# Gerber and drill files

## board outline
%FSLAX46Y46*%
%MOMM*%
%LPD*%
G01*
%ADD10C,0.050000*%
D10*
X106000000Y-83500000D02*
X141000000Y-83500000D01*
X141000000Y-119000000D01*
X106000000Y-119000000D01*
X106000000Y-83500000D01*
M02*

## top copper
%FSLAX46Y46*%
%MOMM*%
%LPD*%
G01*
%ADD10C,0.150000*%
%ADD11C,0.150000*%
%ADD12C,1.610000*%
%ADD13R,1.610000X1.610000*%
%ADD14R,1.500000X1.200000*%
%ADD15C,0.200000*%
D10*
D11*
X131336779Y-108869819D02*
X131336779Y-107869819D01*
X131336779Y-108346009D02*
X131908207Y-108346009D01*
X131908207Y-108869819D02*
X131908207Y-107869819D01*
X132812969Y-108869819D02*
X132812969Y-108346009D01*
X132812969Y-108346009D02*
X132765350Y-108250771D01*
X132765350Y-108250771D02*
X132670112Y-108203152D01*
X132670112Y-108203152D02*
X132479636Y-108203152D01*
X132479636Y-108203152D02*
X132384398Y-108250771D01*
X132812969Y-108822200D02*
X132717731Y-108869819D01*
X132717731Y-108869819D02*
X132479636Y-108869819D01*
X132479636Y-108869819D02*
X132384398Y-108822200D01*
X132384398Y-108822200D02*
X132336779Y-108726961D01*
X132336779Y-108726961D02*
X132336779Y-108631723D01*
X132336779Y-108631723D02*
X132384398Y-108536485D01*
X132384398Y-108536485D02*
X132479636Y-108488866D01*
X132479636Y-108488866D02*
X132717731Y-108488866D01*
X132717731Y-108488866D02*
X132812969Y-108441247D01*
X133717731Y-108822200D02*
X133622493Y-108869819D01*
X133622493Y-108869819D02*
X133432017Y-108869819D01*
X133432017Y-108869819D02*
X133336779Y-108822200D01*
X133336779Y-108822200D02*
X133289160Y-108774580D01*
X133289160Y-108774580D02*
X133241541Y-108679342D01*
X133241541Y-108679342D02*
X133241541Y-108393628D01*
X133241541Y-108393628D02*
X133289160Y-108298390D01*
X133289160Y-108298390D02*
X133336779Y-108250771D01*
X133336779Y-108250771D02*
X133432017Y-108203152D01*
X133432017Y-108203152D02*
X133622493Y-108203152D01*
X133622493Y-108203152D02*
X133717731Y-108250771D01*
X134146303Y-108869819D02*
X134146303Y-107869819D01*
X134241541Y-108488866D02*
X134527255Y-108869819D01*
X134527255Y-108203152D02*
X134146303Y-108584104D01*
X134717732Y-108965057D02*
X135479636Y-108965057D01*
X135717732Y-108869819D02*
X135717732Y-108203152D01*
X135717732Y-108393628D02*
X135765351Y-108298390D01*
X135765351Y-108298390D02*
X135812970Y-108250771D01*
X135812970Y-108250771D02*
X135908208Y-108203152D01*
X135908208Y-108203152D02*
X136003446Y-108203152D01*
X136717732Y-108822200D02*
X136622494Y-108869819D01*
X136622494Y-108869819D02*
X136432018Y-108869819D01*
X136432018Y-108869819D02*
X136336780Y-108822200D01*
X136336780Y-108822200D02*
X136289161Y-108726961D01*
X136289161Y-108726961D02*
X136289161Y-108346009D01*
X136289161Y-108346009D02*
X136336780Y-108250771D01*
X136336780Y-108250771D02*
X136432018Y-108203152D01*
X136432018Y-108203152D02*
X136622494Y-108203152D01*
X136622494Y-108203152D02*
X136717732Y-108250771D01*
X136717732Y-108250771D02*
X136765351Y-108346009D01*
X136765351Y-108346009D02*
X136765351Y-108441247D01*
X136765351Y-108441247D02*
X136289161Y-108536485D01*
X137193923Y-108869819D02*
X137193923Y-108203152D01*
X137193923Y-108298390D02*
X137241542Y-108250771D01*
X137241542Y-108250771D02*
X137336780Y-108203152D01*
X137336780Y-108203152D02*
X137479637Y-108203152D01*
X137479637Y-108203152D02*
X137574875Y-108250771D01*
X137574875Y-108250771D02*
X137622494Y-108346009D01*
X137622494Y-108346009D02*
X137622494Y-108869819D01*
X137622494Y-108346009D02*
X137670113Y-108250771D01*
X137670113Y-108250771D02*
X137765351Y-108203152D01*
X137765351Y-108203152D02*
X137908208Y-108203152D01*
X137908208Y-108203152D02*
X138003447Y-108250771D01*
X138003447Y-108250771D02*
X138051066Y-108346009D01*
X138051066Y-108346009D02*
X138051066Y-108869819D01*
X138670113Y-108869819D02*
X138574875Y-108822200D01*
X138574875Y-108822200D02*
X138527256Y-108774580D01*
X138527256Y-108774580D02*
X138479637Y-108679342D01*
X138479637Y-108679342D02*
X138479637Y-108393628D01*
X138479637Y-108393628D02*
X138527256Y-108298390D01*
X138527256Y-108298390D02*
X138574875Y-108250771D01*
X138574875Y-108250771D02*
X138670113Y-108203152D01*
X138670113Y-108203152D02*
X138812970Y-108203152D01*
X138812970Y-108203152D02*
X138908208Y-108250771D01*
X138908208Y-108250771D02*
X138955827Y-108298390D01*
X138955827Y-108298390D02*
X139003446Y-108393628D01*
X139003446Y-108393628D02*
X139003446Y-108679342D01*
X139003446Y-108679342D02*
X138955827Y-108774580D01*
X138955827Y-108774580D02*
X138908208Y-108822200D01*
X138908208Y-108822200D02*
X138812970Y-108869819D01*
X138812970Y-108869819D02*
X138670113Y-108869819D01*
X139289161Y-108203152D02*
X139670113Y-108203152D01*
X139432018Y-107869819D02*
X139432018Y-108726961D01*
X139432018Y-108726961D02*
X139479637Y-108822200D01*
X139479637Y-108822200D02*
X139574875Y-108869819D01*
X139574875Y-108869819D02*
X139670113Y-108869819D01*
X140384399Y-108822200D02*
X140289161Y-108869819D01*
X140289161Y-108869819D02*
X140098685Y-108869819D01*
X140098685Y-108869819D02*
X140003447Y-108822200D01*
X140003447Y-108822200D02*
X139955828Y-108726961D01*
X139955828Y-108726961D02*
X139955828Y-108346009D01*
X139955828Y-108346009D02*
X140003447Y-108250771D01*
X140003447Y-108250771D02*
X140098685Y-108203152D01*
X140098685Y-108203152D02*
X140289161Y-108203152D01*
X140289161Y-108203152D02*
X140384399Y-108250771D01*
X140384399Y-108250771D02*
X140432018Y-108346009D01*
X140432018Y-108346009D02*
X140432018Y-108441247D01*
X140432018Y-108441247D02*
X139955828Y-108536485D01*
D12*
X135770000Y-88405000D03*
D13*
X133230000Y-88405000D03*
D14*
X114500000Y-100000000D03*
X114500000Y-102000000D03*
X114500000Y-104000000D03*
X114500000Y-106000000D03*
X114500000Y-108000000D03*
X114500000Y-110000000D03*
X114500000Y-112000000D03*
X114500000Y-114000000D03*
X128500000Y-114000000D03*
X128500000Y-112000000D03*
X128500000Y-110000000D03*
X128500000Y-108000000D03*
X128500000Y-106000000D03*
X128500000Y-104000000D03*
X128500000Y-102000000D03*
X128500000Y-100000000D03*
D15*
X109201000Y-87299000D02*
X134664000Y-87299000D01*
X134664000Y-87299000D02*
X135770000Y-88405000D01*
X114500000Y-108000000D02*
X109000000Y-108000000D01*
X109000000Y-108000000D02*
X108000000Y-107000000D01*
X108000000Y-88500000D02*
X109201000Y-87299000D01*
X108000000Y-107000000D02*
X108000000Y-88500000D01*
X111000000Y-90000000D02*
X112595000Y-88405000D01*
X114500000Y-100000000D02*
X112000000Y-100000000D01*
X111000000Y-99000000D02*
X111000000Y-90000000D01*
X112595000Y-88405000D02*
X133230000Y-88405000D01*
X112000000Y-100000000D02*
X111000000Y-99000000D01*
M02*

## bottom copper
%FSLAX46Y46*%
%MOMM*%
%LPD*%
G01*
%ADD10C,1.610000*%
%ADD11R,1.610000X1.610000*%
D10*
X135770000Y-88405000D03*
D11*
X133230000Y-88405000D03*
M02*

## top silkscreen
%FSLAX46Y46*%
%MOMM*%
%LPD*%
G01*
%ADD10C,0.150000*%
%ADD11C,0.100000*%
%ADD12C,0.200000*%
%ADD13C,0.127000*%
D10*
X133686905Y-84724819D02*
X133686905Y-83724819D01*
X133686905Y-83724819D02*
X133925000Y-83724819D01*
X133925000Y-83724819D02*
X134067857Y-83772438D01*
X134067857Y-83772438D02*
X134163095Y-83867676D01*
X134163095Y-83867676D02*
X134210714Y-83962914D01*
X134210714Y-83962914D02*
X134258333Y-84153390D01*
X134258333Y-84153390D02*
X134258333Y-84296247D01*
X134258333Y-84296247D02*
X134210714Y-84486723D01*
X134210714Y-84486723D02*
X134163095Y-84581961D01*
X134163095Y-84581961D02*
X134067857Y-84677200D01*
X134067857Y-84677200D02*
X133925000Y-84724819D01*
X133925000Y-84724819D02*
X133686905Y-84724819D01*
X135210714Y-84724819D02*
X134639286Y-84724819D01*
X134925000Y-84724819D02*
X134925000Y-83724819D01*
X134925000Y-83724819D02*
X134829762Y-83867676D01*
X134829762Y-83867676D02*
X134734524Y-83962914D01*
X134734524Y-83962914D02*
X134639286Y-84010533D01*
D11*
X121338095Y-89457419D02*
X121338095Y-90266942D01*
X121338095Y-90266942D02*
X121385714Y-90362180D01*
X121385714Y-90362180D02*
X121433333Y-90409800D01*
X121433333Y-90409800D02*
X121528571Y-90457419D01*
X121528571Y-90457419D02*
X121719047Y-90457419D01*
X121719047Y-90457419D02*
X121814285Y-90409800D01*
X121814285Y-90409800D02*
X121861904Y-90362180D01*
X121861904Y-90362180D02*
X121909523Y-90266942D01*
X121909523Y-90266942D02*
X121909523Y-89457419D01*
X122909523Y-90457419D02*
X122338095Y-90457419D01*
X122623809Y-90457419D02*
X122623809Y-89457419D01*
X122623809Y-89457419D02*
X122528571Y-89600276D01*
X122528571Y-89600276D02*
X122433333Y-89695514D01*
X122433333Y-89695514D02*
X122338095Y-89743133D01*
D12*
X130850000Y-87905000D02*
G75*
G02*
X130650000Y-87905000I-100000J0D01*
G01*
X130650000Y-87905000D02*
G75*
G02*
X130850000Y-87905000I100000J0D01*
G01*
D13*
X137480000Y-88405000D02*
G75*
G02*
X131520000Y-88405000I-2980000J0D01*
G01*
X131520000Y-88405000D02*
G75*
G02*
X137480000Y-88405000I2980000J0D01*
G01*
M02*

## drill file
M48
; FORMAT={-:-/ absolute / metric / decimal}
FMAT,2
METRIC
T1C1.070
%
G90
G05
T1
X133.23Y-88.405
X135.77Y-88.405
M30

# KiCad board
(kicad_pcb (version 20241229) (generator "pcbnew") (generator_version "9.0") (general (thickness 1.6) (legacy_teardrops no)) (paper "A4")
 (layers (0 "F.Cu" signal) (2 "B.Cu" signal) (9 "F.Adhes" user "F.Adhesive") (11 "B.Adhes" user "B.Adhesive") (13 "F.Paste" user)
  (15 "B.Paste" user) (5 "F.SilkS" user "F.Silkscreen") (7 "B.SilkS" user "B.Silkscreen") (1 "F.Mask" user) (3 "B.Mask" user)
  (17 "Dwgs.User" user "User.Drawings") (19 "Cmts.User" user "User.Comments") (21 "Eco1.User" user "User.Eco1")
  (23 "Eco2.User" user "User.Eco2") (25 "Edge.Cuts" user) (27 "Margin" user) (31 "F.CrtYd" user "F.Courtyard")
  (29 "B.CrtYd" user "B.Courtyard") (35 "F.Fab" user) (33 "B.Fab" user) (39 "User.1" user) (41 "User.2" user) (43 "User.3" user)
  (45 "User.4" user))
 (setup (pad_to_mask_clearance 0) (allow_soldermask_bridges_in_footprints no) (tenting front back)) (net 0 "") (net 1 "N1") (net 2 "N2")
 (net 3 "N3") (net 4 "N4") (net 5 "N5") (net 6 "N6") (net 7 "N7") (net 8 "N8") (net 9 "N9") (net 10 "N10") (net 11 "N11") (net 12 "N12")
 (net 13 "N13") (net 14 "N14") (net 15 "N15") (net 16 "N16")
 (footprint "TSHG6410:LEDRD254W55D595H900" (layer "F.Cu") (at 134.5 88.405)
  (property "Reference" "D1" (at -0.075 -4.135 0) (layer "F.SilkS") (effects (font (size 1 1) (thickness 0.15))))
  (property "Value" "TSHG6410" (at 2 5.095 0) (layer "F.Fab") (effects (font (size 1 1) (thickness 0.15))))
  (fp_circle (center -3.75 -0.5) (end -3.65 -0.5) (stroke (width 0.2) (type solid)) (fill no) (layer "F.SilkS"))
  (fp_circle (center 0 0) (end 2.98 0) (stroke (width 0.127) (type solid)) (fill no) (layer "F.SilkS"))
  (pad "A" thru_hole circle (at 1.27 0) (size 1.61 1.61) (drill 1.07) (layers "*.Cu" "*.Mask") (remove_unused_layers no) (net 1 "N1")
   (solder_mask_margin 0.102))
  (pad "C" thru_hole rect (at -1.27 0) (size 1.61 1.61) (drill 1.07) (layers "*.Cu" "*.Mask") (remove_unused_layers no) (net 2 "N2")
   (solder_mask_margin 0.102)))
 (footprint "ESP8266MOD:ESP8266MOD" (layer "F.Cu") (at 108.3 85.4)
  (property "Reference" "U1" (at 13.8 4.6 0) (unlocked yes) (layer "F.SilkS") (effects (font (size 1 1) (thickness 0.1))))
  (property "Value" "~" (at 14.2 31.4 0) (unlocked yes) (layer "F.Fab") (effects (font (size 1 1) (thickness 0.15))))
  (pad "1" smd rect (at 6.2 14.6) (size 1.5 1.2) (layers "F.Cu" "F.Mask" "F.Paste") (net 2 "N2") (thermal_bridge_angle 45))
  (pad "2" smd rect (at 6.2 16.6) (size 1.5 1.2) (layers "F.Cu" "F.Mask" "F.Paste") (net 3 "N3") (thermal_bridge_angle 45))
  (pad "3" smd rect (at 6.2 18.6) (size 1.5 1.2) (layers "F.Cu" "F.Mask" "F.Paste") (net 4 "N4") (thermal_bridge_angle 45))
  (pad "4" smd rect (at 6.2 20.6) (size 1.5 1.2) (layers "F.Cu" "F.Mask" "F.Paste") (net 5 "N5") (thermal_bridge_angle 45))
  (pad "5" smd rect (at 6.2 22.6) (size 1.5 1.2) (layers "F.Cu" "F.Mask" "F.Paste") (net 1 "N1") (thermal_bridge_angle 45))
  (pad "6" smd rect (at 6.2 24.6) (size 1.5 1.2) (layers "F.Cu" "F.Mask" "F.Paste") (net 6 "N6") (thermal_bridge_angle 45))
  (pad "7" smd rect (at 6.2 26.6) (size 1.5 1.2) (layers "F.Cu" "F.Mask" "F.Paste") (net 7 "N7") (thermal_bridge_angle 45))
  (pad "8" smd rect (at 6.2 28.6) (size 1.5 1.2) (layers "F.Cu" "F.Mask" "F.Paste") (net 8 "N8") (thermal_bridge_angle 45))
  (pad "9" smd rect (at 20.2 28.6) (size 1.5 1.2) (layers "F.Cu" "F.Mask" "F.Paste") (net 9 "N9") (thermal_bridge_angle 45))
  (pad "10" smd rect (at 20.2 26.6) (size 1.5 1.2) (layers "F.Cu" "F.Mask" "F.Paste") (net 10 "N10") (thermal_bridge_angle 45))
  (pad "11" smd rect (at 20.2 24.6) (size 1.5 1.2) (layers "F.Cu" "F.Mask" "F.Paste") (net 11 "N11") (thermal_bridge_angle 45))
  (pad "12" smd rect (at 20.2 22.6) (size 1.5 1.2) (layers "F.Cu" "F.Mask" "F.Paste") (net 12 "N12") (thermal_bridge_angle 45))
  (pad "13" smd rect (at 20.2 20.6) (size 1.5 1.2) (layers "F.Cu" "F.Mask" "F.Paste") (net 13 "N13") (thermal_bridge_angle 45))
  (pad "14" smd rect (at 20.2 18.6) (size 1.5 1.2) (layers "F.Cu" "F.Mask" "F.Paste") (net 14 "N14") (thermal_bridge_angle 45))
  (pad "15" smd rect (at 20.2 16.6) (size 1.5 1.2) (layers "F.Cu" "F.Mask" "F.Paste") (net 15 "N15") (thermal_bridge_angle 45))
  (pad "16" smd rect (at 20.2 14.6) (size 1.5 1.2) (layers "F.Cu" "F.Mask" "F.Paste") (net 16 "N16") (thermal_bridge_angle 45))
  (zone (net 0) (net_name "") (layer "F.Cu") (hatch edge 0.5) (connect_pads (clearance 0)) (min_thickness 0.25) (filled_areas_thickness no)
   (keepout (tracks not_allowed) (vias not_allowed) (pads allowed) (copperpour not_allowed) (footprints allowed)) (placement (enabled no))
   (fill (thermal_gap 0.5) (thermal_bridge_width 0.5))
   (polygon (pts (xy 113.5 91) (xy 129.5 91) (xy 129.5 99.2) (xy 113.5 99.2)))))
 (gr_rect (start 106 83.5) (end 141 119) (stroke (width 0.05) (type default)) (fill no) (layer "Edge.Cuts"))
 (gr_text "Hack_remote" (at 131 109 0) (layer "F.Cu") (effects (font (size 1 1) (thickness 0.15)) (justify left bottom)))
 (segment (start 109.201 87.299) (end 134.664 87.299) (width 0.2) (layer "F.Cu") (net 1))
 (segment (start 134.664 87.299) (end 135.77 88.405) (width 0.2) (layer "F.Cu") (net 1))
 (segment (start 114.5 108) (end 109 108) (width 0.2) (layer "F.Cu") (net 1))
 (segment (start 109 108) (end 108 107) (width 0.2) (layer "F.Cu") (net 1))
 (segment (start 108 88.5) (end 109.201 87.299) (width 0.2) (layer "F.Cu") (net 1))
 (segment (start 108 107) (end 108 88.5) (width 0.2) (layer "F.Cu") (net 1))
 (segment (start 111 90) (end 112.595 88.405) (width 0.2) (layer "F.Cu") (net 2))
 (segment (start 114.5 100) (end 112 100) (width 0.2) (layer "F.Cu") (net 2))
 (segment (start 111 99) (end 111 90) (width 0.2) (layer "F.Cu") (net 2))
 (segment (start 112.595 88.405) (end 133.23 88.405) (width 0.2) (layer "F.Cu") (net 2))
 (segment (start 112 100) (end 111 99) (width 0.2) (layer "F.Cu") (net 2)))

